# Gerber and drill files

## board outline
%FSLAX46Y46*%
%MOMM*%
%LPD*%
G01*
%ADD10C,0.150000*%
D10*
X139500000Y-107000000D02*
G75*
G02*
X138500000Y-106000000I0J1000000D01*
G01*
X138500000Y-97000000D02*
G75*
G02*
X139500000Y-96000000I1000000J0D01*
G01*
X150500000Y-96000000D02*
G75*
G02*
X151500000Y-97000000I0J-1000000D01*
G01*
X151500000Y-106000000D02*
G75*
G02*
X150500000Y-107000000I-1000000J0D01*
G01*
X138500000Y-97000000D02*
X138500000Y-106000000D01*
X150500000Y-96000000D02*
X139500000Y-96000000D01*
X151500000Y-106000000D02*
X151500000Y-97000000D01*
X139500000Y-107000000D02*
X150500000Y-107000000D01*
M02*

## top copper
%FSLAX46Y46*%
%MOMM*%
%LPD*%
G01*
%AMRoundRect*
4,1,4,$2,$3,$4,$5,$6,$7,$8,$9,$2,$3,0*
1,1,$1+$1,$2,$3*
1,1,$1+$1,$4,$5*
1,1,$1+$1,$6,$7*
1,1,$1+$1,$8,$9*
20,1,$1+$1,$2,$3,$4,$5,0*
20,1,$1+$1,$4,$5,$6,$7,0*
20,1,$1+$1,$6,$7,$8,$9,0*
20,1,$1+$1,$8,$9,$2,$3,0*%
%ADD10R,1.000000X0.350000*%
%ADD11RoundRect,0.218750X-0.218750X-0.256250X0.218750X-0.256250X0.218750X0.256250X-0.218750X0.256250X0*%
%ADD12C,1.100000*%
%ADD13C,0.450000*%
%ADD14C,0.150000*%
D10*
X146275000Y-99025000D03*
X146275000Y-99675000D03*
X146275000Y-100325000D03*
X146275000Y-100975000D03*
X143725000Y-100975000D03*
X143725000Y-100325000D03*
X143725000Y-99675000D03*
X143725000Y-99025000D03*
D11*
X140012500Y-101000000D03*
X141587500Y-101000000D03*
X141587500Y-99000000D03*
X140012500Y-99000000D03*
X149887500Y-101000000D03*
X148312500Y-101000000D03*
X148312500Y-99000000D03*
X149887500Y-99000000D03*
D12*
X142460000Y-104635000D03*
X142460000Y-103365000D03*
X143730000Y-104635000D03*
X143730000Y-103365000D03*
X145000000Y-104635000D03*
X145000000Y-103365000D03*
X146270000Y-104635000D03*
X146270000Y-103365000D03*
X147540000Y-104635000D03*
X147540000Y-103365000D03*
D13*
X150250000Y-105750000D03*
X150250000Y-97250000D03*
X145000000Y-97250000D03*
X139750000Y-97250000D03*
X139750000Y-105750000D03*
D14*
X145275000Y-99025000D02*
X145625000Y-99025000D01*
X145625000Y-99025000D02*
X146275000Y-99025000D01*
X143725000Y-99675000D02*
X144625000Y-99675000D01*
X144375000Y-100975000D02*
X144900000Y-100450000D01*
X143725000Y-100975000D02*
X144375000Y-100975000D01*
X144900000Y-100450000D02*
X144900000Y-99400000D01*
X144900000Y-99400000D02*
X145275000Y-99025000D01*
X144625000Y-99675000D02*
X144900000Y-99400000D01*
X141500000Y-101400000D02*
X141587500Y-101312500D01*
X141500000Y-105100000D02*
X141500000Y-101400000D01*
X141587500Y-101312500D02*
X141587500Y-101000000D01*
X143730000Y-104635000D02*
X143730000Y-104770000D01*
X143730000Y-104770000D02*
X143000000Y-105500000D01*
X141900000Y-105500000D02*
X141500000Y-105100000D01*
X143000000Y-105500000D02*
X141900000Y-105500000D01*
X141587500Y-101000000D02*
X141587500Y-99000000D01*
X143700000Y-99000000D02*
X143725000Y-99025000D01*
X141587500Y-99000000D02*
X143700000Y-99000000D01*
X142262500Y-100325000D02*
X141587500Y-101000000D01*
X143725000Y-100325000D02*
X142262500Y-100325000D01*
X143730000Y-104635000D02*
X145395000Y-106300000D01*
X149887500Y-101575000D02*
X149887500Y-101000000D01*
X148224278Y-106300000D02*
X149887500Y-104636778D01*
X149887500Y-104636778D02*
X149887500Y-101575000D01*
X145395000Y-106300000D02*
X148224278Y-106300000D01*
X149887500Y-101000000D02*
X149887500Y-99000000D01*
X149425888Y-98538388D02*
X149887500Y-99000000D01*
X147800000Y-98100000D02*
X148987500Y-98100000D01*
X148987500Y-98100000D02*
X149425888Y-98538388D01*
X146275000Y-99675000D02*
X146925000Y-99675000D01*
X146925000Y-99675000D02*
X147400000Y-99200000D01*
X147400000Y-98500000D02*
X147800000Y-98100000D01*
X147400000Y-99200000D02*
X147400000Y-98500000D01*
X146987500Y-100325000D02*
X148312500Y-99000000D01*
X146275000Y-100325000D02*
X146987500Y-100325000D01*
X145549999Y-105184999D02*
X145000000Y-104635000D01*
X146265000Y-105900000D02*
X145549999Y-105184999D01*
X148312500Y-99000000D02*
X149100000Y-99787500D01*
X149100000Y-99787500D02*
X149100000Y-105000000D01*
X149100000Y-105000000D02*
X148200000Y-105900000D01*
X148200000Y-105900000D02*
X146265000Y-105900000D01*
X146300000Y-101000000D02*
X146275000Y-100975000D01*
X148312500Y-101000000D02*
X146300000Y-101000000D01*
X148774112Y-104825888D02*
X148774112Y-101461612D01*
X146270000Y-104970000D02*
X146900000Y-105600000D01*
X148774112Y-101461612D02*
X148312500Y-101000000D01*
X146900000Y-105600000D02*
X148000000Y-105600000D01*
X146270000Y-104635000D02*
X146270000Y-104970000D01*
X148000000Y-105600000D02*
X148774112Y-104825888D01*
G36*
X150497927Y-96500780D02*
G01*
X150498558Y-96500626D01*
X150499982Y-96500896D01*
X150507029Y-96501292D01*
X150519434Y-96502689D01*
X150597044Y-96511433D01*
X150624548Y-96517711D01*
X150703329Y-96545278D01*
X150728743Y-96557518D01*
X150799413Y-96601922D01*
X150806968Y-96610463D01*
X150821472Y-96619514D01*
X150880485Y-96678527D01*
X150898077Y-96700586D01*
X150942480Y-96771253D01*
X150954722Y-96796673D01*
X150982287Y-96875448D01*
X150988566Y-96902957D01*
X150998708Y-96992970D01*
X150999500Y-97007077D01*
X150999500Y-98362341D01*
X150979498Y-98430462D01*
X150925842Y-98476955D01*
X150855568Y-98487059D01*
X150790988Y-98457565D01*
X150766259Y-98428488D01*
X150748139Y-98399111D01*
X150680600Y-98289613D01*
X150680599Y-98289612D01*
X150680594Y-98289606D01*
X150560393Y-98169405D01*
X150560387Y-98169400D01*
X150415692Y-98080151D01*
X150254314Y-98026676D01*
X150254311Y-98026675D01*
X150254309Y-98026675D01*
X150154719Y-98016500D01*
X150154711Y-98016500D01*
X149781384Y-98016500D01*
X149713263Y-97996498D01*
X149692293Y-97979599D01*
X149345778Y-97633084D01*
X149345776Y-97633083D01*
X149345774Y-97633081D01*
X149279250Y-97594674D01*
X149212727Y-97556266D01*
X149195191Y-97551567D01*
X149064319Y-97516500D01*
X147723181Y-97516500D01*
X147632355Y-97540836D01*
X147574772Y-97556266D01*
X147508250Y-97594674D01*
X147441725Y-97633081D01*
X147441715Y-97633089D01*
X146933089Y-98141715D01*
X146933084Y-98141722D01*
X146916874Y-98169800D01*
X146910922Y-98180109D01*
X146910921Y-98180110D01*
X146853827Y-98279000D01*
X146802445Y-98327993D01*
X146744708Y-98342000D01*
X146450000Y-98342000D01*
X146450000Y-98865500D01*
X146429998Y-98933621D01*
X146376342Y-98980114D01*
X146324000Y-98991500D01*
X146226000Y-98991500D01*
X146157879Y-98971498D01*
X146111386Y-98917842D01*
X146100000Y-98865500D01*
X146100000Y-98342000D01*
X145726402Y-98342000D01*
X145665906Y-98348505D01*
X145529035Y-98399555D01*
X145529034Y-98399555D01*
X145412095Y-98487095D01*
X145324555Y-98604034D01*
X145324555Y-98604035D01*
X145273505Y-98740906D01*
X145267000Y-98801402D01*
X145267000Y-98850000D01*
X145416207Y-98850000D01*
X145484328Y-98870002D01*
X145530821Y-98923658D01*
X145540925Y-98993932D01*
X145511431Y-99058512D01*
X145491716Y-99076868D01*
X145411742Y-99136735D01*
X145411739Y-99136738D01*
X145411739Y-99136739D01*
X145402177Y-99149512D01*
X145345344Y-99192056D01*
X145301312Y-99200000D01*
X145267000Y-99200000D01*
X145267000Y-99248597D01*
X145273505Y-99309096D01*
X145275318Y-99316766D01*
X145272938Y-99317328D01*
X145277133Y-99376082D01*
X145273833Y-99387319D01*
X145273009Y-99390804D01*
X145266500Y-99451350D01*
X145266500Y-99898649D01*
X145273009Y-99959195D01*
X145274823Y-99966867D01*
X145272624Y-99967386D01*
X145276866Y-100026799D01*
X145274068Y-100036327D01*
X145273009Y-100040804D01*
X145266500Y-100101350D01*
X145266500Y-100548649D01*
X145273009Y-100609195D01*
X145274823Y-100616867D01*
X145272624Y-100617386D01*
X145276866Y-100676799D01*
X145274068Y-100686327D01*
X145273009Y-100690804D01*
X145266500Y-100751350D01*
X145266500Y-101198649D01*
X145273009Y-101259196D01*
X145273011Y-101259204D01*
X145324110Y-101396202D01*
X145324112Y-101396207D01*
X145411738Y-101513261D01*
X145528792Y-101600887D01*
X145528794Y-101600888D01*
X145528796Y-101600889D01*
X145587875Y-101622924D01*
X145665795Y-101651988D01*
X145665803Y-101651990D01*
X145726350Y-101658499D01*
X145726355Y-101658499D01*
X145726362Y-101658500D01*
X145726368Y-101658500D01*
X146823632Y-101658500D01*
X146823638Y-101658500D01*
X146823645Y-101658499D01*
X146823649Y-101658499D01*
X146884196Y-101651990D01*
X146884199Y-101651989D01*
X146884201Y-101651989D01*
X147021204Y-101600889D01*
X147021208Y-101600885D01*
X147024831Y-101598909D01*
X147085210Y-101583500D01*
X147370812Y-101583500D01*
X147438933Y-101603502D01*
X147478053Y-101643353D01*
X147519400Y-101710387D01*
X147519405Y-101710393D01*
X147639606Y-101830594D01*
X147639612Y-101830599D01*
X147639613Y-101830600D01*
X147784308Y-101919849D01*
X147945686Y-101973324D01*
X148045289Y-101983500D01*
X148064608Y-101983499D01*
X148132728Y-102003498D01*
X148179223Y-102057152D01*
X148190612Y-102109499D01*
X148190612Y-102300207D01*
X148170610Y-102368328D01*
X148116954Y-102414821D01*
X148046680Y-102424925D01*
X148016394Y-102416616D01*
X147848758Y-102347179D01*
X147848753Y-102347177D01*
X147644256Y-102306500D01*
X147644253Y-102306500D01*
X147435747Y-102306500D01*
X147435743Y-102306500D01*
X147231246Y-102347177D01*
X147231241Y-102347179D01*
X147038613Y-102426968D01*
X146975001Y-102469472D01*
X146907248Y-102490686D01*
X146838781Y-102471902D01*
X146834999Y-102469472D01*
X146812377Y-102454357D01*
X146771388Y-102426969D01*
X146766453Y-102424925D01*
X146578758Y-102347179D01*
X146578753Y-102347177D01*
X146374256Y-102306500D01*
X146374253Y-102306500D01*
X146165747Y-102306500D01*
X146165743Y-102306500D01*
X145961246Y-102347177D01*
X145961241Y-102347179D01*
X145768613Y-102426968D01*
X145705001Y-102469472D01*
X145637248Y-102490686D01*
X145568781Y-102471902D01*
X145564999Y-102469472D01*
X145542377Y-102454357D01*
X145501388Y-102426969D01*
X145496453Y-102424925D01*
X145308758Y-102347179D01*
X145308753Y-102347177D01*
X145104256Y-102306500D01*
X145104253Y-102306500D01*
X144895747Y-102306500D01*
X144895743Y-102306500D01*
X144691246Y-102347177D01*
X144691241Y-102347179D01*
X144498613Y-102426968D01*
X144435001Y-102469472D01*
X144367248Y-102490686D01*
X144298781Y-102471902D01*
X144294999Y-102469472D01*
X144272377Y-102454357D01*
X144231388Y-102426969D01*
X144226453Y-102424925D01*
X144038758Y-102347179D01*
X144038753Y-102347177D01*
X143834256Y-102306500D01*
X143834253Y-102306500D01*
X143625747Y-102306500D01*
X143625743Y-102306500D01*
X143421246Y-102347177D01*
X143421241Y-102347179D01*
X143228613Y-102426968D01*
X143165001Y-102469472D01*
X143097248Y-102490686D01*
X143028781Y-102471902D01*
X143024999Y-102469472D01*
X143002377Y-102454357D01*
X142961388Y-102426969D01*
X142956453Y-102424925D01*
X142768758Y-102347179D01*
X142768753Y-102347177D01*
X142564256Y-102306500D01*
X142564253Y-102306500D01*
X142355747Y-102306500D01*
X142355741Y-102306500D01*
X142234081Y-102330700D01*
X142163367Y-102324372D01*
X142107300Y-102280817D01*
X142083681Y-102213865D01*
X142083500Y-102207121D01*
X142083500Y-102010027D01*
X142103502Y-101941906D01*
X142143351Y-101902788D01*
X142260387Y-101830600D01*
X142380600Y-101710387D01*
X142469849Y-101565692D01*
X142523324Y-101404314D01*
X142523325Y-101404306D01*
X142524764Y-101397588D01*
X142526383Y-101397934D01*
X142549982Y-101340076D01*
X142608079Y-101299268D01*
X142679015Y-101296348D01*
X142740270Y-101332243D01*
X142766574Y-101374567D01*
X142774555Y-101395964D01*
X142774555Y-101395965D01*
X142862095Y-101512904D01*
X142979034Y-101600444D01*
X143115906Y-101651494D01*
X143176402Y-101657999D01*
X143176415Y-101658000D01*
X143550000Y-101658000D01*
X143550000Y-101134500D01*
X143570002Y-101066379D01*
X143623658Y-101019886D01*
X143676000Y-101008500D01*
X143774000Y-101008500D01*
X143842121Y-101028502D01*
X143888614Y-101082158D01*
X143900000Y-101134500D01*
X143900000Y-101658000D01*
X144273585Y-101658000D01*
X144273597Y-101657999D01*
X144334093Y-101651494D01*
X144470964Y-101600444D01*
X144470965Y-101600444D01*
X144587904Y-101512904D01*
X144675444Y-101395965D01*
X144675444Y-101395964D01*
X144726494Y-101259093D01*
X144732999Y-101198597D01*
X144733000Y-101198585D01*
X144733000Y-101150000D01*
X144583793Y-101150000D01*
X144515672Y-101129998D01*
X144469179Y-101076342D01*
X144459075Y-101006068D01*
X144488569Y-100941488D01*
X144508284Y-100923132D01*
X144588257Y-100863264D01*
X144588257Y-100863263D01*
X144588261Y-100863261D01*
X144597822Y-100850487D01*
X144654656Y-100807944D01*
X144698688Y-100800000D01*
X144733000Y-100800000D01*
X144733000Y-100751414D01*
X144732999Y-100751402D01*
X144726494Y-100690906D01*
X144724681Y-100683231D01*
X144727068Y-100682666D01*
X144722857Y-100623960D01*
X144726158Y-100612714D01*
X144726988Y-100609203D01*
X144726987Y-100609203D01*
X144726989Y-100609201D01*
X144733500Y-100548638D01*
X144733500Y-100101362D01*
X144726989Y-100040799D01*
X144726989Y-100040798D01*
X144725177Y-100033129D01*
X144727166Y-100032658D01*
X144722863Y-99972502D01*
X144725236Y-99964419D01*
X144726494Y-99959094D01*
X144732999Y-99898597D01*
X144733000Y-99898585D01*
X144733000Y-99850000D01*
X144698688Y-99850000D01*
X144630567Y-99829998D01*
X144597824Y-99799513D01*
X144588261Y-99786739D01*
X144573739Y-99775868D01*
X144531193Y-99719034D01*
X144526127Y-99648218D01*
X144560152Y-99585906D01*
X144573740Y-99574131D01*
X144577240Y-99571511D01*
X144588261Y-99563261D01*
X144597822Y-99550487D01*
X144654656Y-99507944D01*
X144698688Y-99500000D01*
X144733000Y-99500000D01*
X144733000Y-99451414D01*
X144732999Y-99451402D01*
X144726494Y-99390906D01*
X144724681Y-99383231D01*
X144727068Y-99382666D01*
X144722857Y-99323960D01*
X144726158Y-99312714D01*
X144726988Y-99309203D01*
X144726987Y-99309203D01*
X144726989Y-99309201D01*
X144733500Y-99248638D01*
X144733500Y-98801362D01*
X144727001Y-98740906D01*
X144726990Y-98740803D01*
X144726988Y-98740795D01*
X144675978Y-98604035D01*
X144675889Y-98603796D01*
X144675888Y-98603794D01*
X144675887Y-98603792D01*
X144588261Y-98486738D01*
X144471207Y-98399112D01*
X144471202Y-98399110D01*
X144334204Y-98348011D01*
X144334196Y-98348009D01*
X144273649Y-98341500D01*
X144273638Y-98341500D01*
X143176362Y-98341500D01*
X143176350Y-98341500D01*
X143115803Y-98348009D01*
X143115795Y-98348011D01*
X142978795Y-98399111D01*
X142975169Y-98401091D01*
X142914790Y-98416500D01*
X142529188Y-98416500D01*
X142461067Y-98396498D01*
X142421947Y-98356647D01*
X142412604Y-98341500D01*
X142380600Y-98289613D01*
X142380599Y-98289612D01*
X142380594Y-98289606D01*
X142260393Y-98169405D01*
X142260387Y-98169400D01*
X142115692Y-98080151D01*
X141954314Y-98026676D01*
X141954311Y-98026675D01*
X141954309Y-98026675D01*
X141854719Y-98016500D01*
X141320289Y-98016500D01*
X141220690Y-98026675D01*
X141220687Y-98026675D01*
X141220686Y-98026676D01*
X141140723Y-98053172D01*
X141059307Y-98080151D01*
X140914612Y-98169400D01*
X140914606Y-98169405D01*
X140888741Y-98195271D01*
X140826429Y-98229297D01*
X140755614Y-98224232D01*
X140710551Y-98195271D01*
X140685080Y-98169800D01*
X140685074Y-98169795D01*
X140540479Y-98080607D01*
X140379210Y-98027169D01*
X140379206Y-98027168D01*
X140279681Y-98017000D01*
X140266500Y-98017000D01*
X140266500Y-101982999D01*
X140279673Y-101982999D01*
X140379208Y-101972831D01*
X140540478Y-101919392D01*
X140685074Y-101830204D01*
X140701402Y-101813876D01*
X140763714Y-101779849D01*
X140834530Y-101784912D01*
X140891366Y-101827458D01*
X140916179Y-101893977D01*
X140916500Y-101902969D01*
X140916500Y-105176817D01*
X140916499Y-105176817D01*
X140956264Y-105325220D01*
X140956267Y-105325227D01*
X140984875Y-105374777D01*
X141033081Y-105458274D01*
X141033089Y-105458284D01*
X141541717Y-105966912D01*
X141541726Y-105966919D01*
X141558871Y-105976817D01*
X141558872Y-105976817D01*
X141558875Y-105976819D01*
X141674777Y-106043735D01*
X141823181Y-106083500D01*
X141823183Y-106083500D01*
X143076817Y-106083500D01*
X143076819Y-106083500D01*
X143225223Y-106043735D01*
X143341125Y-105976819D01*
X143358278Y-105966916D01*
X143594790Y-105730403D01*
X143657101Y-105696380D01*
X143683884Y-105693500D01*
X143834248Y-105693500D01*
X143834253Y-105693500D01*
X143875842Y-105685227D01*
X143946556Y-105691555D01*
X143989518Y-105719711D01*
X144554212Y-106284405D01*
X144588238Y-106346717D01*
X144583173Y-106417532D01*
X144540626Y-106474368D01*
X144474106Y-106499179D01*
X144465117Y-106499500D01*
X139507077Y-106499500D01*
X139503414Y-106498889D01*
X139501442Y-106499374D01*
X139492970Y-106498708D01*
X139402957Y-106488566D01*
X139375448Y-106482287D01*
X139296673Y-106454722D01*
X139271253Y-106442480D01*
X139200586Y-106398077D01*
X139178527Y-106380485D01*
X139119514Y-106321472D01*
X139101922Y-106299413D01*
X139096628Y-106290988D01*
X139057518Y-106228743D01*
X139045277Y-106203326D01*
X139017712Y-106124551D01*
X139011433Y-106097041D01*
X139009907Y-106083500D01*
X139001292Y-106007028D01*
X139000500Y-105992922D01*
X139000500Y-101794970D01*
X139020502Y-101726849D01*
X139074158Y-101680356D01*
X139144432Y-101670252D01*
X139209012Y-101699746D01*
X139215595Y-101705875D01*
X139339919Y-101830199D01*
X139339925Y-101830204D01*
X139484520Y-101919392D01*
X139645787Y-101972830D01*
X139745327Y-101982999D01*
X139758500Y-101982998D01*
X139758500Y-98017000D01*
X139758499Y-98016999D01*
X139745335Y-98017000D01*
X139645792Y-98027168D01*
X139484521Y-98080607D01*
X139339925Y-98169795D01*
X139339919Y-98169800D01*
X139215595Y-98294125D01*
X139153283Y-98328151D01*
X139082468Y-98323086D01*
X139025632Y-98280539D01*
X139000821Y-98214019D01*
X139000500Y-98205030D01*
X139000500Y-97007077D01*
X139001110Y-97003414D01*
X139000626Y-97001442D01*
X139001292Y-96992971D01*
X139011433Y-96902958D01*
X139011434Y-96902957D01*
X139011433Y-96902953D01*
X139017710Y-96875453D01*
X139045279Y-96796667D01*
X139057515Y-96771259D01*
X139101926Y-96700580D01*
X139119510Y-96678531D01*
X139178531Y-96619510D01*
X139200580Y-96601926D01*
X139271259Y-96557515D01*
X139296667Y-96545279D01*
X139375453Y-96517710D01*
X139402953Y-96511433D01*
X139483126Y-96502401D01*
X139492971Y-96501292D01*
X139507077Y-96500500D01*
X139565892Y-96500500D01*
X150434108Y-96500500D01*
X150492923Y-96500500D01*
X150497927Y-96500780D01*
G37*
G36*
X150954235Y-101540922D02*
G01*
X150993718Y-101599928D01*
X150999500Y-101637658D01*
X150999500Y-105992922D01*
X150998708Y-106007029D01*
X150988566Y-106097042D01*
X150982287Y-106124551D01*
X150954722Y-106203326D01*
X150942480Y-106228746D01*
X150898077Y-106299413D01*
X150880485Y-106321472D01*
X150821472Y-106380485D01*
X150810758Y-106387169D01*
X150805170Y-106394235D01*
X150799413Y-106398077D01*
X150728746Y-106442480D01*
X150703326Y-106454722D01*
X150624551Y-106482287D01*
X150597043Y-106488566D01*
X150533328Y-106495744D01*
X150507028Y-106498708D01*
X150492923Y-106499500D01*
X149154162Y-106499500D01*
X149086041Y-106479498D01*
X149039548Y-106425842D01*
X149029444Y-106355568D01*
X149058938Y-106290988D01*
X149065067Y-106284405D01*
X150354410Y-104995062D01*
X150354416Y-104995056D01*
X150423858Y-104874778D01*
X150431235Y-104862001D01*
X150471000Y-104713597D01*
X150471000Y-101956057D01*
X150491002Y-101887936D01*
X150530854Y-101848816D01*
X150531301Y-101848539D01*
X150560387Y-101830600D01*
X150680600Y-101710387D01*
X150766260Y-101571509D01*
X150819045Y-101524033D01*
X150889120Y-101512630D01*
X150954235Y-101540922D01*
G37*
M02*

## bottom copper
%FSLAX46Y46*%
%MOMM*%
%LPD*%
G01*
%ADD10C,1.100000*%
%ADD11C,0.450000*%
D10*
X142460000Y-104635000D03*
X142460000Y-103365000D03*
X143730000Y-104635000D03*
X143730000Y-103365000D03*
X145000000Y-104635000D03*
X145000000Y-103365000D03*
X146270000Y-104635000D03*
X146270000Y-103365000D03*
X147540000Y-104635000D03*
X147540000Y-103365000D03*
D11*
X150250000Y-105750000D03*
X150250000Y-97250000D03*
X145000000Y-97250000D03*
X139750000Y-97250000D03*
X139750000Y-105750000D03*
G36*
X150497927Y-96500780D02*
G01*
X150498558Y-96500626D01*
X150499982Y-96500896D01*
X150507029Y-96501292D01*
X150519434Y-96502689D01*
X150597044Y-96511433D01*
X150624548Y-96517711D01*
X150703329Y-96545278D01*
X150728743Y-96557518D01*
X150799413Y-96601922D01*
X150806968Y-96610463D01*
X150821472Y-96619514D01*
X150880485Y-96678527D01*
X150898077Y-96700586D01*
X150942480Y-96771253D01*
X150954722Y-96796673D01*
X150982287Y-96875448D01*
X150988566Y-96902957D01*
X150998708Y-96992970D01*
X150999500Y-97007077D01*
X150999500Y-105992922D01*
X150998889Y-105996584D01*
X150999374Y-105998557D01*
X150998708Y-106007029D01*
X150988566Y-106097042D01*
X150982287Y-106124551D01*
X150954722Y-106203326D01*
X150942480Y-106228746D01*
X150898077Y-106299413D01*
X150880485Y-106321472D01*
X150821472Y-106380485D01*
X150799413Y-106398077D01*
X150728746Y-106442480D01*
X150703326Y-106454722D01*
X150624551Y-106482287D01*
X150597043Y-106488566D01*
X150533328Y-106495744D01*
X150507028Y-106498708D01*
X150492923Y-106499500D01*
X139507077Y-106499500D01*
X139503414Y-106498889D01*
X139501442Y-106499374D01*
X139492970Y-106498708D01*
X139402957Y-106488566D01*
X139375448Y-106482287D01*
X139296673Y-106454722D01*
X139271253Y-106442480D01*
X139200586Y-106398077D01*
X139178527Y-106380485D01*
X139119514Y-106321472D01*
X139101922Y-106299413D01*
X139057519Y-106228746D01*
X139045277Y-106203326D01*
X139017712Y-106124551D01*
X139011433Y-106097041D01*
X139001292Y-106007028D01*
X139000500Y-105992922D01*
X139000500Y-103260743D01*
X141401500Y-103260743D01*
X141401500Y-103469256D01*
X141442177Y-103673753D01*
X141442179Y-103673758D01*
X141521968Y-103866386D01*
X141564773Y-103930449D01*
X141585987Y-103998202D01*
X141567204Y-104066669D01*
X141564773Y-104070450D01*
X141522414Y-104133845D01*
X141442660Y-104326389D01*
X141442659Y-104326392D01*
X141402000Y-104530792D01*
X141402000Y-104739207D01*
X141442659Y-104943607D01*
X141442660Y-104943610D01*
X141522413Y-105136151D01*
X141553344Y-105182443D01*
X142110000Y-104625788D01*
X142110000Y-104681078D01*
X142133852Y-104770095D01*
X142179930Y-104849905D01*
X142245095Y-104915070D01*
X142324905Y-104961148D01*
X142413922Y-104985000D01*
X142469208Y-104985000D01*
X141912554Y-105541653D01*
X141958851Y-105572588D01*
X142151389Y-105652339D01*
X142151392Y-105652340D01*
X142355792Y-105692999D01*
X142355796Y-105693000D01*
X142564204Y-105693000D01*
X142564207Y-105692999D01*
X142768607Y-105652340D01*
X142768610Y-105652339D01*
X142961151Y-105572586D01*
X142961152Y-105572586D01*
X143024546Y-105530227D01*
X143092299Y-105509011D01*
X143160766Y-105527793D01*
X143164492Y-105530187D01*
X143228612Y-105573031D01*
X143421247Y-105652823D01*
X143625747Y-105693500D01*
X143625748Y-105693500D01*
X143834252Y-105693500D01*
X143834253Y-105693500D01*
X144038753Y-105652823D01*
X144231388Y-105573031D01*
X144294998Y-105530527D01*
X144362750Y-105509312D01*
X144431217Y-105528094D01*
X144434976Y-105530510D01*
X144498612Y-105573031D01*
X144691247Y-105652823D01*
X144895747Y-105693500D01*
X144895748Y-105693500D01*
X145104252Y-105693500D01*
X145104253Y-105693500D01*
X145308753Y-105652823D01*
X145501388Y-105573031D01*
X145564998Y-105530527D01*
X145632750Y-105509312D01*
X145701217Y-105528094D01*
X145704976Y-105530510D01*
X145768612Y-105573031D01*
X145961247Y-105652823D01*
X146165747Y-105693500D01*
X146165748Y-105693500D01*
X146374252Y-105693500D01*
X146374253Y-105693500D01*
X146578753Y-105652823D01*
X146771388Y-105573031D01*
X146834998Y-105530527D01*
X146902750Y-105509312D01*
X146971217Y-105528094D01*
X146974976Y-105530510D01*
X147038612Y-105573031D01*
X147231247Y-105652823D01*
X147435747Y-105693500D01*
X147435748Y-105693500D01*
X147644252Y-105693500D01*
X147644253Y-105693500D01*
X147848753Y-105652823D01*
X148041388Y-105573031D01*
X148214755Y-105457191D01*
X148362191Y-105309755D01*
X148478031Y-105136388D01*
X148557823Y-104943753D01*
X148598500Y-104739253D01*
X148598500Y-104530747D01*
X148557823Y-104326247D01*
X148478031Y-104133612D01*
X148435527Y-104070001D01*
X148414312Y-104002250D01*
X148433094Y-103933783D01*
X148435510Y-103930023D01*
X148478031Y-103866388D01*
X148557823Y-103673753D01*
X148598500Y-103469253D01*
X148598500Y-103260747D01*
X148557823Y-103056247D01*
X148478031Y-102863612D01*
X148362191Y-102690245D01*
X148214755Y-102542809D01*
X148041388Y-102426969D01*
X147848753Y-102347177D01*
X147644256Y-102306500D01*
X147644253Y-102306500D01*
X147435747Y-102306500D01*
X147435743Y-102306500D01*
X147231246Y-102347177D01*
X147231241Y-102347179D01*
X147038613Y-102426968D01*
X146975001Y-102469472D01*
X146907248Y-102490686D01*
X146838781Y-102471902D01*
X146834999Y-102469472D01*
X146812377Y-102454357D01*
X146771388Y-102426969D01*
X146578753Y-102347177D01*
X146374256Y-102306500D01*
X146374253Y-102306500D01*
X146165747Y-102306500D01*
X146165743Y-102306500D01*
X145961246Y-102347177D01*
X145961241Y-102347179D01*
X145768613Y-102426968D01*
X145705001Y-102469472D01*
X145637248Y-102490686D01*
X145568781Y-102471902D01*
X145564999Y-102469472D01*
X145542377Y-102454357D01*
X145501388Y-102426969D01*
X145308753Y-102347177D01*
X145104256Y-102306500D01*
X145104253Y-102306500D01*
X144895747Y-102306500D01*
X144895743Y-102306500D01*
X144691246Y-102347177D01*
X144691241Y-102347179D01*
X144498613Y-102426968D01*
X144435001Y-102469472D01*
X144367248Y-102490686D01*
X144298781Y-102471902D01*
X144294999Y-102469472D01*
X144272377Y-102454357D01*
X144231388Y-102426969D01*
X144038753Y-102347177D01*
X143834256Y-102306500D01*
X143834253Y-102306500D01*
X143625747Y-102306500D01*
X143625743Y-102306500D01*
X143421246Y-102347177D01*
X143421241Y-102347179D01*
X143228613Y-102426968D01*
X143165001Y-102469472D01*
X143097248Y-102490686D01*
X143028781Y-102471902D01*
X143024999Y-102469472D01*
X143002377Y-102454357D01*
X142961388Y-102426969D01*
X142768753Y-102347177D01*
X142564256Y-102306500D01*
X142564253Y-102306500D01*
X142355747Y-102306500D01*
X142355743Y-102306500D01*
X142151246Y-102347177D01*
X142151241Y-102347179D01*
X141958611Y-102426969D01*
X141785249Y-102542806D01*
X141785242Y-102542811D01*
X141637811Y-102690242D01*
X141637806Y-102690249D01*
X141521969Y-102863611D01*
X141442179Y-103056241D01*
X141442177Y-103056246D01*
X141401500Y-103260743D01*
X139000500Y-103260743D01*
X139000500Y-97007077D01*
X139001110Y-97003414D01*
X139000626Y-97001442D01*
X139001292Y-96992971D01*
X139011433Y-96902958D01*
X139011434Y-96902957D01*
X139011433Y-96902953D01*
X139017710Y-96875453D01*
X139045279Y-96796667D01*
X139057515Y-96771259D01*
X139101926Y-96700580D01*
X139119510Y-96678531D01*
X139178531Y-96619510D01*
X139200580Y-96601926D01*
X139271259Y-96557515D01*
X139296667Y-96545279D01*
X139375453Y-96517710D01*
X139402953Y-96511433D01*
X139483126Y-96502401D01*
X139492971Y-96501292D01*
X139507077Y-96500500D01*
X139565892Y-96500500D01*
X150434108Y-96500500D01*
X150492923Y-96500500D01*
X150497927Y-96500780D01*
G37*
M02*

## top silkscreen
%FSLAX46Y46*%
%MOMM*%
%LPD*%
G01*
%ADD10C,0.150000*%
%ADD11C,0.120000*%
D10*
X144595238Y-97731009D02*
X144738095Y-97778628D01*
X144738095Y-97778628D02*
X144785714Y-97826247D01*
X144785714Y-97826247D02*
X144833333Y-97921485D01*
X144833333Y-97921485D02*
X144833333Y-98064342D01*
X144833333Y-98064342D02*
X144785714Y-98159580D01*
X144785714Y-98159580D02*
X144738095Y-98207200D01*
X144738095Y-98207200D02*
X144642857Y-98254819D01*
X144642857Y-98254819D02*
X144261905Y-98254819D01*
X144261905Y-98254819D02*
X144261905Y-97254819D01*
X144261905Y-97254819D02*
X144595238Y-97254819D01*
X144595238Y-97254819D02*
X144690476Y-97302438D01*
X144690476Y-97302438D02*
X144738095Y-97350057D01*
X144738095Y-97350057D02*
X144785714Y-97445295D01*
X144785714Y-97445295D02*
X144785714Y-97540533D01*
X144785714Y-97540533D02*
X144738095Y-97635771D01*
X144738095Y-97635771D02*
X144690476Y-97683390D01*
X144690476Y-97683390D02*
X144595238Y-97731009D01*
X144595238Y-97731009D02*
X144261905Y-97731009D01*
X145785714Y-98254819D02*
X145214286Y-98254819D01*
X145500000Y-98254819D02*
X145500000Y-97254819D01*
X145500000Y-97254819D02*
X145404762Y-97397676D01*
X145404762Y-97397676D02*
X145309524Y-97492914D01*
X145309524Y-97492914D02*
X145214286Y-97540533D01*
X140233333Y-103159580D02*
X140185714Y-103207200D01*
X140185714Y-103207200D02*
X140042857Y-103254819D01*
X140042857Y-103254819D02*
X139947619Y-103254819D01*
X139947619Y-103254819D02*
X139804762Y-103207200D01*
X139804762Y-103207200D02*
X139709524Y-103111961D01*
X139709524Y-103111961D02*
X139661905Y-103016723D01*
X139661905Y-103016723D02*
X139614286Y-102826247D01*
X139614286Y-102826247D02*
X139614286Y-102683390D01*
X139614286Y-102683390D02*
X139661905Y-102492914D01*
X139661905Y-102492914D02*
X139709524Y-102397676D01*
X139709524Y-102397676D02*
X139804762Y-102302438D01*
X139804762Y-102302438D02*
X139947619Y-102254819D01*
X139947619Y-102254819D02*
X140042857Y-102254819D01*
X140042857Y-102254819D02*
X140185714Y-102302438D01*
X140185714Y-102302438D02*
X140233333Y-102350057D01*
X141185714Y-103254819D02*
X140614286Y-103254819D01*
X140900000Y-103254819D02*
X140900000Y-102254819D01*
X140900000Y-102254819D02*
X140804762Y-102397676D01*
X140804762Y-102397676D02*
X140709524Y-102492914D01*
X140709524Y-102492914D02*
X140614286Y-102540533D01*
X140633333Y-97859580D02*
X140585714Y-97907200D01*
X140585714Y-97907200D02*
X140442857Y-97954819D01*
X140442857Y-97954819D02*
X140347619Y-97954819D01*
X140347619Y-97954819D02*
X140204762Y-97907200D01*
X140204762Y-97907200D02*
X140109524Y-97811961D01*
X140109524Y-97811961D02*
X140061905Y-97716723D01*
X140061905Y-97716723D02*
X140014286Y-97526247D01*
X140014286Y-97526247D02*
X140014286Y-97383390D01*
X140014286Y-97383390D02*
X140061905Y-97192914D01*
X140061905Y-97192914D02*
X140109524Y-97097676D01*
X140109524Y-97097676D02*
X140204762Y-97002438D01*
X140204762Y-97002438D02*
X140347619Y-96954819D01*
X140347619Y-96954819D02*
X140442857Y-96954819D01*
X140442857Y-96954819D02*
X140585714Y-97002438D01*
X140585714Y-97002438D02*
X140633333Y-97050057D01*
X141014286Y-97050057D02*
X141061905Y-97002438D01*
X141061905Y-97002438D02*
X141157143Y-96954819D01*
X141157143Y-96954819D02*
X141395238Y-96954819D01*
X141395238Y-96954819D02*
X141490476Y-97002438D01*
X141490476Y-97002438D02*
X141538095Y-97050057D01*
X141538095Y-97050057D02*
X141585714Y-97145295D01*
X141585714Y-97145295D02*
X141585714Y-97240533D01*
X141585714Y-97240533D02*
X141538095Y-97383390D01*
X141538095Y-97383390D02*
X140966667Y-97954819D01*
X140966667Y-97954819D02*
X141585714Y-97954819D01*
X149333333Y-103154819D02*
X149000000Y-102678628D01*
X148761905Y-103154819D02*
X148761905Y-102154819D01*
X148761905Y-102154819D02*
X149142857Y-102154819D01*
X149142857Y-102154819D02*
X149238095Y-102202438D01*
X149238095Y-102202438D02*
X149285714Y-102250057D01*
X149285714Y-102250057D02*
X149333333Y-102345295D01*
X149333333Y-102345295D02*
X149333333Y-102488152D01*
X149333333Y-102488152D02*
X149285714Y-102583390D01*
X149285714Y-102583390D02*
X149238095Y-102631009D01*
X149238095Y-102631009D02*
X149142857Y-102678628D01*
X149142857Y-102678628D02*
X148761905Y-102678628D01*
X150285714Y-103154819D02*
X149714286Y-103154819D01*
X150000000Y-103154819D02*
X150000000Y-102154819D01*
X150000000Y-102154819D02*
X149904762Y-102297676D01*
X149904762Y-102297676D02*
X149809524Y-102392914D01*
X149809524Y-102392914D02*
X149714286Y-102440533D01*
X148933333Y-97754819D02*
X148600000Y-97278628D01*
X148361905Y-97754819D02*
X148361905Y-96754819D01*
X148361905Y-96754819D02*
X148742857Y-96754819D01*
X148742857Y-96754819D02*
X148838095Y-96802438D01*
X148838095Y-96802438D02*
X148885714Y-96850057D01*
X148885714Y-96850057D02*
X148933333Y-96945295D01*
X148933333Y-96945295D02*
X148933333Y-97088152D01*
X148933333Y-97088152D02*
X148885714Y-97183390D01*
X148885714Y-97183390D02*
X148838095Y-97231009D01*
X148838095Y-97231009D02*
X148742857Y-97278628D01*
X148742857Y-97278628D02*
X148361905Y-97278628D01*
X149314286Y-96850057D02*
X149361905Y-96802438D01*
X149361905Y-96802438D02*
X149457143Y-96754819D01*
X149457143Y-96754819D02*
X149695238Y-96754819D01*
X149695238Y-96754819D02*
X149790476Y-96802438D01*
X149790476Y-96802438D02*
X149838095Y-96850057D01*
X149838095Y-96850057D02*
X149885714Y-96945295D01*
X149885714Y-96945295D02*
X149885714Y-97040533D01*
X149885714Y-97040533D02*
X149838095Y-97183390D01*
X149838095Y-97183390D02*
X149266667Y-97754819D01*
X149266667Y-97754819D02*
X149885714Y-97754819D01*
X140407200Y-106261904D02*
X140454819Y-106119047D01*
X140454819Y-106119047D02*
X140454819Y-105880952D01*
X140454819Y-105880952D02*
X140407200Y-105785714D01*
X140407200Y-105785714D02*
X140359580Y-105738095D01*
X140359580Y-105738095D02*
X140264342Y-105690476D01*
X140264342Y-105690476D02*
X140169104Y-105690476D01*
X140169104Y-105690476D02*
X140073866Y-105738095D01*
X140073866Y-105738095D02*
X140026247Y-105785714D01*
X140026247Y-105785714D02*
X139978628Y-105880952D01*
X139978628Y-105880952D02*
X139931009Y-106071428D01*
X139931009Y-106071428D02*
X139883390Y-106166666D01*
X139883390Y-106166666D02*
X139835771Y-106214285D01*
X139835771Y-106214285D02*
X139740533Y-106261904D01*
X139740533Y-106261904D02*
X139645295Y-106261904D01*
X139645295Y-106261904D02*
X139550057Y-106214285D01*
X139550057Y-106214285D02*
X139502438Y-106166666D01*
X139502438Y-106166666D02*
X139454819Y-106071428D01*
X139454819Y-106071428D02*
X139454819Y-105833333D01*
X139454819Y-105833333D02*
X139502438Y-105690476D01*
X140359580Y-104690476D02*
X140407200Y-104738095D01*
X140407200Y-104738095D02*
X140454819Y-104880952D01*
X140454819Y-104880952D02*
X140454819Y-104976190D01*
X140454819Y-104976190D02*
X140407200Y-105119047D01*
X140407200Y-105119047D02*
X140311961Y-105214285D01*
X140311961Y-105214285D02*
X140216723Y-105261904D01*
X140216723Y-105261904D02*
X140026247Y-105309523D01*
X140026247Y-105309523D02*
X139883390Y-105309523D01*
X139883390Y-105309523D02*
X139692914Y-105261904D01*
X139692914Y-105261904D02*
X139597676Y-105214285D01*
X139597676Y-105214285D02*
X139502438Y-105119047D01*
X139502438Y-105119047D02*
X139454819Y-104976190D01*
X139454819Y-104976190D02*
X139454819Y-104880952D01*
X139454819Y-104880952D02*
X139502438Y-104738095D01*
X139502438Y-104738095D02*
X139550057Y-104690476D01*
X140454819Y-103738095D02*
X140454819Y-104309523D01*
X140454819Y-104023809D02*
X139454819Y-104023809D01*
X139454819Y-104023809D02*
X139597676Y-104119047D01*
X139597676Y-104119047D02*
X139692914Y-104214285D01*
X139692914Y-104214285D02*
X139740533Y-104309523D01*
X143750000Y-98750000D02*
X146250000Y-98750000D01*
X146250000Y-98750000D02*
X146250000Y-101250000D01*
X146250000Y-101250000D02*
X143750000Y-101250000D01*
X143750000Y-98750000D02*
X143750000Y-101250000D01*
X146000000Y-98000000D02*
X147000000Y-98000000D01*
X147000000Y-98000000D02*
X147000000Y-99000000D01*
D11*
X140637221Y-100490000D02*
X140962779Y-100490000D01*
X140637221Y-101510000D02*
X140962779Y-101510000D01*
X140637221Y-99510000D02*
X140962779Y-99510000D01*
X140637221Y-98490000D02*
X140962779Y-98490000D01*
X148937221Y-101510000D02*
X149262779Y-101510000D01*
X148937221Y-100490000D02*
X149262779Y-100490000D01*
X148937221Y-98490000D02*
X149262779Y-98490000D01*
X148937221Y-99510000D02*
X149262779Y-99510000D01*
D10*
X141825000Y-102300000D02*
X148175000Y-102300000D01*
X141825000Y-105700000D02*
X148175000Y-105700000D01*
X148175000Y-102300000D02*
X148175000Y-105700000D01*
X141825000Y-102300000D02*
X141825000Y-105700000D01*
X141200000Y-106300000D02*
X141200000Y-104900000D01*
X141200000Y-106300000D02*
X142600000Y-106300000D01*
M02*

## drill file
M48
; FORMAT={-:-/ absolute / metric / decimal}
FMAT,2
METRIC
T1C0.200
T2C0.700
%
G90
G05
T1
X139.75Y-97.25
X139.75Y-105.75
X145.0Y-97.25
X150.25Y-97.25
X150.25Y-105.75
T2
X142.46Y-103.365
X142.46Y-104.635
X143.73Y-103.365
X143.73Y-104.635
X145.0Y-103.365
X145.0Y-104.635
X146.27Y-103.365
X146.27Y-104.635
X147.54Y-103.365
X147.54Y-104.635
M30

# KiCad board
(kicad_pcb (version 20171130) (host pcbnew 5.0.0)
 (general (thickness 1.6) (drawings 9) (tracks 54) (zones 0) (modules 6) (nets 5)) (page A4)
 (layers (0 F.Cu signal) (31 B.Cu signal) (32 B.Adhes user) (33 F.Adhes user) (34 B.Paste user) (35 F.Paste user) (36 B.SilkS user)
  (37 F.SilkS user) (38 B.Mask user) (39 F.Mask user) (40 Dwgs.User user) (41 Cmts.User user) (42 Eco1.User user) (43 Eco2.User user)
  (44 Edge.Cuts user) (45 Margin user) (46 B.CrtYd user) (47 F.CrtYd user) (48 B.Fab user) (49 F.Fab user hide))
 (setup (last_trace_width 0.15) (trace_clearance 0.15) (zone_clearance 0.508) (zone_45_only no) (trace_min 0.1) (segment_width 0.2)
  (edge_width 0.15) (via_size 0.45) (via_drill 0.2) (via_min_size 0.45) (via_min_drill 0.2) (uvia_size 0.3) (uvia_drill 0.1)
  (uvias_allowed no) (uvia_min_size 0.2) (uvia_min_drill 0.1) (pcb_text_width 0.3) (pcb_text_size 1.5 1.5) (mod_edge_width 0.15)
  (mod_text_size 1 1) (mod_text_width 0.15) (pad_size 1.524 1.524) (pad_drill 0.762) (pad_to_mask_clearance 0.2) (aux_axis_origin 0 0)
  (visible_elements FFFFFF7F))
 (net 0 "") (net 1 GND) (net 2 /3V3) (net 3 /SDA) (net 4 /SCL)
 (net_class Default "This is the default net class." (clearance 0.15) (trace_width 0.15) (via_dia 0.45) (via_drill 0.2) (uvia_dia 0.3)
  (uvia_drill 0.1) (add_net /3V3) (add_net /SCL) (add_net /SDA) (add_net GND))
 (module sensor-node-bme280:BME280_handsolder (layer F.Cu) (at 145 100)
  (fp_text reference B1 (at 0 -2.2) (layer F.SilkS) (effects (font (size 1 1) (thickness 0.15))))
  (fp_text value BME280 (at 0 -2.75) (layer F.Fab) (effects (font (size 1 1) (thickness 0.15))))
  (fp_line (start -1.25 -1.25) (end 1.25 -1.25) (layer F.SilkS) (width 0.15))
  (fp_line (start 1.25 -1.25) (end 1.25 1.25) (layer F.SilkS) (width 0.15))
  (fp_line (start 1.25 1.25) (end -1.25 1.25) (layer F.SilkS) (width 0.15))
  (fp_line (start -1.25 -1.25) (end -1.25 1.25) (layer F.SilkS) (width 0.15))
  (fp_line (start 1 -2) (end 2 -2) (layer F.SilkS) (width 0.15))
  (fp_line (start 2 -2) (end 2 -1) (layer F.SilkS) (width 0.15))
  (pad 1 smd rect (at 1.275 -0.975) (size 1 0.35) (layers F.Cu F.Paste F.Mask) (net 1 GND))
  (pad 2 smd rect (at 1.275 -0.325) (size 1 0.35) (layers F.Cu F.Paste F.Mask) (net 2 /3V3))
  (pad 3 smd rect (at 1.275 0.325) (size 1 0.35) (layers F.Cu F.Paste F.Mask) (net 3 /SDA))
  (pad 4 smd rect (at 1.275 0.975) (size 1 0.35) (layers F.Cu F.Paste F.Mask) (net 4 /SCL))
  (pad 5 smd rect (at -1.275 0.975) (size 1 0.35) (layers F.Cu F.Paste F.Mask) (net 1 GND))
  (pad 6 smd rect (at -1.275 0.325) (size 1 0.35) (layers F.Cu F.Paste F.Mask) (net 2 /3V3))
  (pad 7 smd rect (at -1.275 -0.325) (size 1 0.35) (layers F.Cu F.Paste F.Mask) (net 1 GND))
  (pad 8 smd rect (at -1.275 -0.975) (size 1 0.35) (layers F.Cu F.Paste F.Mask) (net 2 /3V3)))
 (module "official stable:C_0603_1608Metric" (layer F.Cu) (at 140.8 101)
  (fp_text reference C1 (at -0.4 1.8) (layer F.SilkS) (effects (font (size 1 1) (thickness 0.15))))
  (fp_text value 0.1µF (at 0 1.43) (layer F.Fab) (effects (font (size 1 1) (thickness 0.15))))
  (fp_line (start -0.162779 -0.51) (end 0.162779 -0.51) (layer F.SilkS) (width 0.12))
  (fp_line (start -0.162779 0.51) (end 0.162779 0.51) (layer F.SilkS) (width 0.12))
  (pad 1 smd roundrect (at -0.7875 0) (size 0.875 0.95) (layers F.Cu F.Paste F.Mask) (roundrect_rratio 0.25) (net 1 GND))
  (pad 2 smd roundrect (at 0.7875 0) (size 0.875 0.95) (layers F.Cu F.Paste F.Mask) (roundrect_rratio 0.25) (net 2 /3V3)))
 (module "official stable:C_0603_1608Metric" (layer F.Cu) (at 140.8 99)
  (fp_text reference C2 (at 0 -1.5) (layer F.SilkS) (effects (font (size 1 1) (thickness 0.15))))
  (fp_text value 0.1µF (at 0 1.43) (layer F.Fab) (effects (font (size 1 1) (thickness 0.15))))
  (fp_line (start -0.162779 0.51) (end 0.162779 0.51) (layer F.SilkS) (width 0.12))
  (fp_line (start -0.162779 -0.51) (end 0.162779 -0.51) (layer F.SilkS) (width 0.12))
  (pad 2 smd roundrect (at 0.7875 0) (size 0.875 0.95) (layers F.Cu F.Paste F.Mask) (roundrect_rratio 0.25) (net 2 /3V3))
  (pad 1 smd roundrect (at -0.7875 0) (size 0.875 0.95) (layers F.Cu F.Paste F.Mask) (roundrect_rratio 0.25) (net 1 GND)))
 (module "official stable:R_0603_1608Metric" (layer F.Cu) (at 149.1 101)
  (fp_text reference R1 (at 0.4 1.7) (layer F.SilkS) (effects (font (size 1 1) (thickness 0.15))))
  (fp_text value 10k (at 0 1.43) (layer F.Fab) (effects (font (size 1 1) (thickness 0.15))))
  (fp_line (start -0.162779 0.51) (end 0.162779 0.51) (layer F.SilkS) (width 0.12))
  (fp_line (start -0.162779 -0.51) (end 0.162779 -0.51) (layer F.SilkS) (width 0.12))
  (pad 2 smd roundrect (at 0.7875 0) (size 0.875 0.95) (layers F.Cu F.Paste F.Mask) (roundrect_rratio 0.25) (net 2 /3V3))
  (pad 1 smd roundrect (at -0.7875 0) (size 0.875 0.95) (layers F.Cu F.Paste F.Mask) (roundrect_rratio 0.25) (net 4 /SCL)))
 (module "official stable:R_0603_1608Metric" (layer F.Cu) (at 149.1 99)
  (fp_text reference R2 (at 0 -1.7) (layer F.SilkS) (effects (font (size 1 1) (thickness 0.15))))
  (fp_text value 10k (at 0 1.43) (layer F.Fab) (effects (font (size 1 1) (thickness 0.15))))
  (fp_line (start -0.162779 -0.51) (end 0.162779 -0.51) (layer F.SilkS) (width 0.12))
  (fp_line (start -0.162779 0.51) (end 0.162779 0.51) (layer F.SilkS) (width 0.12))
  (pad 1 smd roundrect (at -0.7875 0) (size 0.875 0.95) (layers F.Cu F.Paste F.Mask) (roundrect_rratio 0.25) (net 3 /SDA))
  (pad 2 smd roundrect (at 0.7875 0) (size 0.875 0.95) (layers F.Cu F.Paste F.Mask) (roundrect_rratio 0.25) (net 2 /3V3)))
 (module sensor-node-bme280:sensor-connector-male (layer F.Cu) (at 145 104)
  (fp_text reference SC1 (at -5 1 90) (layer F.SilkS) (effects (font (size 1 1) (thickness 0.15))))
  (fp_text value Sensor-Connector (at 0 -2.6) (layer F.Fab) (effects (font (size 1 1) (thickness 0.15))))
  (fp_line (start -3.175 -1.7) (end 3.175 -1.7) (layer F.SilkS) (width 0.15))
  (fp_line (start -3.175 1.7) (end 3.175 1.7) (layer F.SilkS) (width 0.15))
  (fp_line (start 3.175 -1.7) (end 3.175 1.7) (layer F.SilkS) (width 0.15))
  (fp_line (start -3.175 -1.7) (end -3.175 1.7) (layer F.SilkS) (width 0.15))
  (fp_line (start -3.8 2.3) (end -3.8 0.9) (layer F.SilkS) (width 0.15))
  (fp_line (start -3.8 2.3) (end -2.4 2.3) (layer F.SilkS) (width 0.15))
  (pad 1 thru_hole circle (at -2.54 0.635) (size 1.1 1.1) (drill 0.7) (layers *.Cu *.Mask) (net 1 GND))
  (pad 2 thru_hole circle (at -2.54 -0.635) (size 1.1 1.1) (drill 0.7) (layers *.Cu *.Mask))
  (pad 3 thru_hole circle (at -1.27 0.635) (size 1.1 1.1) (drill 0.7) (layers *.Cu *.Mask) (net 2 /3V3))
  (pad 4 thru_hole circle (at -1.27 -0.635) (size 1.1 1.1) (drill 0.7) (layers *.Cu *.Mask))
  (pad 5 thru_hole circle (at 0 0.635) (size 1.1 1.1) (drill 0.7) (layers *.Cu *.Mask) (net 3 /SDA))
  (pad 6 thru_hole circle (at 0 -0.635) (size 1.1 1.1) (drill 0.7) (layers *.Cu *.Mask))
  (pad 7 thru_hole circle (at 1.27 0.635) (size 1.1 1.1) (drill 0.7) (layers *.Cu *.Mask) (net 4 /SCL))
  (pad 8 thru_hole circle (at 1.27 -0.635) (size 1.1 1.1) (drill 0.7) (layers *.Cu *.Mask))
  (pad 9 thru_hole circle (at 2.54 0.635) (size 1.1 1.1) (drill 0.7) (layers *.Cu *.Mask))
  (pad 10 thru_hole circle (at 2.54 -0.635) (size 1.1 1.1) (drill 0.7) (layers *.Cu *.Mask)))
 (gr_arc (start 139.5 106) (end 138.5 106) (angle -90) (layer Edge.Cuts) (width 0.15))
 (gr_arc (start 139.5 97) (end 139.5 96) (angle -90) (layer Edge.Cuts) (width 0.15))
 (gr_arc (start 150.5 97) (end 151.5 97) (angle -90) (layer Edge.Cuts) (width 0.15))
 (gr_arc (start 150.5 106) (end 150.5 107) (angle -90) (layer Edge.Cuts) (width 0.15))
 (gr_line (start 138.5 97) (end 138.5 106) (layer Edge.Cuts) (width 0.15))
 (gr_line (start 150.5 96) (end 139.5 96) (layer Edge.Cuts) (width 0.15))
 (gr_line (start 151.5 106) (end 151.5 97) (layer Edge.Cuts) (width 0.15))
 (gr_line (start 139.5 107) (end 150.5 107) (layer Edge.Cuts) (width 0.15))
 (segment (start 145.275 99.025) (end 145.625 99.025) (width 0.15) (layer F.Cu) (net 1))
 (segment (start 145.625 99.025) (end 146.275 99.025) (width 0.15) (layer F.Cu) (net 1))
 (segment (start 143.725 99.675) (end 144.625 99.675) (width 0.15) (layer F.Cu) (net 1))
 (segment (start 144.375 100.975) (end 144.9 100.45) (width 0.15) (layer F.Cu) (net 1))
 (segment (start 143.725 100.975) (end 144.375 100.975) (width 0.15) (layer F.Cu) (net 1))
 (segment (start 144.9 100.45) (end 144.9 99.4) (width 0.15) (layer F.Cu) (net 1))
 (segment (start 144.9 99.4) (end 145.275 99.025) (width 0.15) (layer F.Cu) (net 1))
 (segment (start 144.625 99.675) (end 144.9 99.4) (width 0.15) (layer F.Cu) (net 1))
 (via (at 150.25 105.75) (size 0.45) (drill 0.2) (layers F.Cu B.Cu) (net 1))
 (via (at 150.25 97.25) (size 0.45) (drill 0.2) (layers F.Cu B.Cu) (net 1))
 (via (at 145 97.25) (size 0.45) (drill 0.2) (layers F.Cu B.Cu) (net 1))
 (via (at 139.75 97.25) (size 0.45) (drill 0.2) (layers F.Cu B.Cu) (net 1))
 (via (at 139.75 105.75) (size 0.45) (drill 0.2) (layers F.Cu B.Cu) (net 1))
 (segment (start 141.5 101.4) (end 141.5875 101.3125) (width 0.15) (layer F.Cu) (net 2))
 (segment (start 141.5 105.1) (end 141.5 101.4) (width 0.15) (layer F.Cu) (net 2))
 (segment (start 141.5875 101.3125) (end 141.5875 101) (width 0.15) (layer F.Cu) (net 2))
 (segment (start 143.73 104.635) (end 143.73 104.77) (width 0.15) (layer F.Cu) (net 2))
 (segment (start 143.73 104.77) (end 143 105.5) (width 0.15) (layer F.Cu) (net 2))
 (segment (start 141.9 105.5) (end 141.5 105.1) (width 0.15) (layer F.Cu) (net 2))
 (segment (start 143 105.5) (end 141.9 105.5) (width 0.15) (layer F.Cu) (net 2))
 (segment (start 141.5875 101) (end 141.5875 99) (width 0.15) (layer F.Cu) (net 2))
 (segment (start 143.7 99) (end 143.725 99.025) (width 0.15) (layer F.Cu) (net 2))
 (segment (start 141.5875 99) (end 143.7 99) (width 0.15) (layer F.Cu) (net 2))
 (segment (start 142.2625 100.325) (end 141.5875 101) (width 0.15) (layer F.Cu) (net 2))
 (segment (start 143.725 100.325) (end 142.2625 100.325) (width 0.15) (layer F.Cu) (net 2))
 (segment (start 143.73 104.635) (end 145.395 106.3) (width 0.15) (layer F.Cu) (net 2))
 (segment (start 149.8875 101.575) (end 149.8875 101) (width 0.15) (layer F.Cu) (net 2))
 (segment (start 148.224278 106.3) (end 149.8875 104.636778) (width 0.15) (layer F.Cu) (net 2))
 (segment (start 149.8875 104.636778) (end 149.8875 101.575) (width 0.15) (layer F.Cu) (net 2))
 (segment (start 145.395 106.3) (end 148.224278 106.3) (width 0.15) (layer F.Cu) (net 2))
 (segment (start 149.8875 101) (end 149.8875 99) (width 0.15) (layer F.Cu) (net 2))
 (segment (start 149.425888 98.538388) (end 149.8875 99) (width 0.15) (layer F.Cu) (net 2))
 (segment (start 147.8 98.1) (end 148.9875 98.1) (width 0.15) (layer F.Cu) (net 2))
 (segment (start 148.9875 98.1) (end 149.425888 98.538388) (width 0.15) (layer F.Cu) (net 2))
 (segment (start 146.275 99.675) (end 146.925 99.675) (width 0.15) (layer F.Cu) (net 2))
 (segment (start 146.925 99.675) (end 147.4 99.2) (width 0.15) (layer F.Cu) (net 2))
 (segment (start 147.4 98.5) (end 147.8 98.1) (width 0.15) (layer F.Cu) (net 2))
 (segment (start 147.4 99.2) (end 147.4 98.5) (width 0.15) (layer F.Cu) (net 2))
 (segment (start 146.9875 100.325) (end 148.3125 99) (width 0.15) (layer F.Cu) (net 3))
 (segment (start 146.275 100.325) (end 146.9875 100.325) (width 0.15) (layer F.Cu) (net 3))
 (segment (start 145.549999 105.184999) (end 145 104.635) (width 0.15) (layer F.Cu) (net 3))
 (segment (start 146.265 105.9) (end 145.549999 105.184999) (width 0.15) (layer F.Cu) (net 3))
 (segment (start 148.3125 99) (end 149.1 99.7875) (width 0.15) (layer F.Cu) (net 3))
 (segment (start 149.1 99.7875) (end 149.1 105) (width 0.15) (layer F.Cu) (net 3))
 (segment (start 149.1 105) (end 148.2 105.9) (width 0.15) (layer F.Cu) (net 3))
 (segment (start 148.2 105.9) (end 146.265 105.9) (width 0.15) (layer F.Cu) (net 3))
 (segment (start 146.3 101) (end 146.275 100.975) (width 0.15) (layer F.Cu) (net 4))
 (segment (start 148.3125 101) (end 146.3 101) (width 0.15) (layer F.Cu) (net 4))
 (segment (start 148.774112 104.825888) (end 148.774112 101.461612) (width 0.15) (layer F.Cu) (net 4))
 (segment (start 146.27 104.97) (end 146.9 105.6) (width 0.15) (layer F.Cu) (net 4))
 (segment (start 148.774112 101.461612) (end 148.3125 101) (width 0.15) (layer F.Cu) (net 4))
 (segment (start 146.9 105.6) (end 148 105.6) (width 0.15) (layer F.Cu) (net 4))
 (segment (start 146.27 104.635) (end 146.27 104.97) (width 0.15) (layer F.Cu) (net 4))
 (segment (start 148 105.6) (end 148.774112 104.825888) (width 0.15) (layer F.Cu) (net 4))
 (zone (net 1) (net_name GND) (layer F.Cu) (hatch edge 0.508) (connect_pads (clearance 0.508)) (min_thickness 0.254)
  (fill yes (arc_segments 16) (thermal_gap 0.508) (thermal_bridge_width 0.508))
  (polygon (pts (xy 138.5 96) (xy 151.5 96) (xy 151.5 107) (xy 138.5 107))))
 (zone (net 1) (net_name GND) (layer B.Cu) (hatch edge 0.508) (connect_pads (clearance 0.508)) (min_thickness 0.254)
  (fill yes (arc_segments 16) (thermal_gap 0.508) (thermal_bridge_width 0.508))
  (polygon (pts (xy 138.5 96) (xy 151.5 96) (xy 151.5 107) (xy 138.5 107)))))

